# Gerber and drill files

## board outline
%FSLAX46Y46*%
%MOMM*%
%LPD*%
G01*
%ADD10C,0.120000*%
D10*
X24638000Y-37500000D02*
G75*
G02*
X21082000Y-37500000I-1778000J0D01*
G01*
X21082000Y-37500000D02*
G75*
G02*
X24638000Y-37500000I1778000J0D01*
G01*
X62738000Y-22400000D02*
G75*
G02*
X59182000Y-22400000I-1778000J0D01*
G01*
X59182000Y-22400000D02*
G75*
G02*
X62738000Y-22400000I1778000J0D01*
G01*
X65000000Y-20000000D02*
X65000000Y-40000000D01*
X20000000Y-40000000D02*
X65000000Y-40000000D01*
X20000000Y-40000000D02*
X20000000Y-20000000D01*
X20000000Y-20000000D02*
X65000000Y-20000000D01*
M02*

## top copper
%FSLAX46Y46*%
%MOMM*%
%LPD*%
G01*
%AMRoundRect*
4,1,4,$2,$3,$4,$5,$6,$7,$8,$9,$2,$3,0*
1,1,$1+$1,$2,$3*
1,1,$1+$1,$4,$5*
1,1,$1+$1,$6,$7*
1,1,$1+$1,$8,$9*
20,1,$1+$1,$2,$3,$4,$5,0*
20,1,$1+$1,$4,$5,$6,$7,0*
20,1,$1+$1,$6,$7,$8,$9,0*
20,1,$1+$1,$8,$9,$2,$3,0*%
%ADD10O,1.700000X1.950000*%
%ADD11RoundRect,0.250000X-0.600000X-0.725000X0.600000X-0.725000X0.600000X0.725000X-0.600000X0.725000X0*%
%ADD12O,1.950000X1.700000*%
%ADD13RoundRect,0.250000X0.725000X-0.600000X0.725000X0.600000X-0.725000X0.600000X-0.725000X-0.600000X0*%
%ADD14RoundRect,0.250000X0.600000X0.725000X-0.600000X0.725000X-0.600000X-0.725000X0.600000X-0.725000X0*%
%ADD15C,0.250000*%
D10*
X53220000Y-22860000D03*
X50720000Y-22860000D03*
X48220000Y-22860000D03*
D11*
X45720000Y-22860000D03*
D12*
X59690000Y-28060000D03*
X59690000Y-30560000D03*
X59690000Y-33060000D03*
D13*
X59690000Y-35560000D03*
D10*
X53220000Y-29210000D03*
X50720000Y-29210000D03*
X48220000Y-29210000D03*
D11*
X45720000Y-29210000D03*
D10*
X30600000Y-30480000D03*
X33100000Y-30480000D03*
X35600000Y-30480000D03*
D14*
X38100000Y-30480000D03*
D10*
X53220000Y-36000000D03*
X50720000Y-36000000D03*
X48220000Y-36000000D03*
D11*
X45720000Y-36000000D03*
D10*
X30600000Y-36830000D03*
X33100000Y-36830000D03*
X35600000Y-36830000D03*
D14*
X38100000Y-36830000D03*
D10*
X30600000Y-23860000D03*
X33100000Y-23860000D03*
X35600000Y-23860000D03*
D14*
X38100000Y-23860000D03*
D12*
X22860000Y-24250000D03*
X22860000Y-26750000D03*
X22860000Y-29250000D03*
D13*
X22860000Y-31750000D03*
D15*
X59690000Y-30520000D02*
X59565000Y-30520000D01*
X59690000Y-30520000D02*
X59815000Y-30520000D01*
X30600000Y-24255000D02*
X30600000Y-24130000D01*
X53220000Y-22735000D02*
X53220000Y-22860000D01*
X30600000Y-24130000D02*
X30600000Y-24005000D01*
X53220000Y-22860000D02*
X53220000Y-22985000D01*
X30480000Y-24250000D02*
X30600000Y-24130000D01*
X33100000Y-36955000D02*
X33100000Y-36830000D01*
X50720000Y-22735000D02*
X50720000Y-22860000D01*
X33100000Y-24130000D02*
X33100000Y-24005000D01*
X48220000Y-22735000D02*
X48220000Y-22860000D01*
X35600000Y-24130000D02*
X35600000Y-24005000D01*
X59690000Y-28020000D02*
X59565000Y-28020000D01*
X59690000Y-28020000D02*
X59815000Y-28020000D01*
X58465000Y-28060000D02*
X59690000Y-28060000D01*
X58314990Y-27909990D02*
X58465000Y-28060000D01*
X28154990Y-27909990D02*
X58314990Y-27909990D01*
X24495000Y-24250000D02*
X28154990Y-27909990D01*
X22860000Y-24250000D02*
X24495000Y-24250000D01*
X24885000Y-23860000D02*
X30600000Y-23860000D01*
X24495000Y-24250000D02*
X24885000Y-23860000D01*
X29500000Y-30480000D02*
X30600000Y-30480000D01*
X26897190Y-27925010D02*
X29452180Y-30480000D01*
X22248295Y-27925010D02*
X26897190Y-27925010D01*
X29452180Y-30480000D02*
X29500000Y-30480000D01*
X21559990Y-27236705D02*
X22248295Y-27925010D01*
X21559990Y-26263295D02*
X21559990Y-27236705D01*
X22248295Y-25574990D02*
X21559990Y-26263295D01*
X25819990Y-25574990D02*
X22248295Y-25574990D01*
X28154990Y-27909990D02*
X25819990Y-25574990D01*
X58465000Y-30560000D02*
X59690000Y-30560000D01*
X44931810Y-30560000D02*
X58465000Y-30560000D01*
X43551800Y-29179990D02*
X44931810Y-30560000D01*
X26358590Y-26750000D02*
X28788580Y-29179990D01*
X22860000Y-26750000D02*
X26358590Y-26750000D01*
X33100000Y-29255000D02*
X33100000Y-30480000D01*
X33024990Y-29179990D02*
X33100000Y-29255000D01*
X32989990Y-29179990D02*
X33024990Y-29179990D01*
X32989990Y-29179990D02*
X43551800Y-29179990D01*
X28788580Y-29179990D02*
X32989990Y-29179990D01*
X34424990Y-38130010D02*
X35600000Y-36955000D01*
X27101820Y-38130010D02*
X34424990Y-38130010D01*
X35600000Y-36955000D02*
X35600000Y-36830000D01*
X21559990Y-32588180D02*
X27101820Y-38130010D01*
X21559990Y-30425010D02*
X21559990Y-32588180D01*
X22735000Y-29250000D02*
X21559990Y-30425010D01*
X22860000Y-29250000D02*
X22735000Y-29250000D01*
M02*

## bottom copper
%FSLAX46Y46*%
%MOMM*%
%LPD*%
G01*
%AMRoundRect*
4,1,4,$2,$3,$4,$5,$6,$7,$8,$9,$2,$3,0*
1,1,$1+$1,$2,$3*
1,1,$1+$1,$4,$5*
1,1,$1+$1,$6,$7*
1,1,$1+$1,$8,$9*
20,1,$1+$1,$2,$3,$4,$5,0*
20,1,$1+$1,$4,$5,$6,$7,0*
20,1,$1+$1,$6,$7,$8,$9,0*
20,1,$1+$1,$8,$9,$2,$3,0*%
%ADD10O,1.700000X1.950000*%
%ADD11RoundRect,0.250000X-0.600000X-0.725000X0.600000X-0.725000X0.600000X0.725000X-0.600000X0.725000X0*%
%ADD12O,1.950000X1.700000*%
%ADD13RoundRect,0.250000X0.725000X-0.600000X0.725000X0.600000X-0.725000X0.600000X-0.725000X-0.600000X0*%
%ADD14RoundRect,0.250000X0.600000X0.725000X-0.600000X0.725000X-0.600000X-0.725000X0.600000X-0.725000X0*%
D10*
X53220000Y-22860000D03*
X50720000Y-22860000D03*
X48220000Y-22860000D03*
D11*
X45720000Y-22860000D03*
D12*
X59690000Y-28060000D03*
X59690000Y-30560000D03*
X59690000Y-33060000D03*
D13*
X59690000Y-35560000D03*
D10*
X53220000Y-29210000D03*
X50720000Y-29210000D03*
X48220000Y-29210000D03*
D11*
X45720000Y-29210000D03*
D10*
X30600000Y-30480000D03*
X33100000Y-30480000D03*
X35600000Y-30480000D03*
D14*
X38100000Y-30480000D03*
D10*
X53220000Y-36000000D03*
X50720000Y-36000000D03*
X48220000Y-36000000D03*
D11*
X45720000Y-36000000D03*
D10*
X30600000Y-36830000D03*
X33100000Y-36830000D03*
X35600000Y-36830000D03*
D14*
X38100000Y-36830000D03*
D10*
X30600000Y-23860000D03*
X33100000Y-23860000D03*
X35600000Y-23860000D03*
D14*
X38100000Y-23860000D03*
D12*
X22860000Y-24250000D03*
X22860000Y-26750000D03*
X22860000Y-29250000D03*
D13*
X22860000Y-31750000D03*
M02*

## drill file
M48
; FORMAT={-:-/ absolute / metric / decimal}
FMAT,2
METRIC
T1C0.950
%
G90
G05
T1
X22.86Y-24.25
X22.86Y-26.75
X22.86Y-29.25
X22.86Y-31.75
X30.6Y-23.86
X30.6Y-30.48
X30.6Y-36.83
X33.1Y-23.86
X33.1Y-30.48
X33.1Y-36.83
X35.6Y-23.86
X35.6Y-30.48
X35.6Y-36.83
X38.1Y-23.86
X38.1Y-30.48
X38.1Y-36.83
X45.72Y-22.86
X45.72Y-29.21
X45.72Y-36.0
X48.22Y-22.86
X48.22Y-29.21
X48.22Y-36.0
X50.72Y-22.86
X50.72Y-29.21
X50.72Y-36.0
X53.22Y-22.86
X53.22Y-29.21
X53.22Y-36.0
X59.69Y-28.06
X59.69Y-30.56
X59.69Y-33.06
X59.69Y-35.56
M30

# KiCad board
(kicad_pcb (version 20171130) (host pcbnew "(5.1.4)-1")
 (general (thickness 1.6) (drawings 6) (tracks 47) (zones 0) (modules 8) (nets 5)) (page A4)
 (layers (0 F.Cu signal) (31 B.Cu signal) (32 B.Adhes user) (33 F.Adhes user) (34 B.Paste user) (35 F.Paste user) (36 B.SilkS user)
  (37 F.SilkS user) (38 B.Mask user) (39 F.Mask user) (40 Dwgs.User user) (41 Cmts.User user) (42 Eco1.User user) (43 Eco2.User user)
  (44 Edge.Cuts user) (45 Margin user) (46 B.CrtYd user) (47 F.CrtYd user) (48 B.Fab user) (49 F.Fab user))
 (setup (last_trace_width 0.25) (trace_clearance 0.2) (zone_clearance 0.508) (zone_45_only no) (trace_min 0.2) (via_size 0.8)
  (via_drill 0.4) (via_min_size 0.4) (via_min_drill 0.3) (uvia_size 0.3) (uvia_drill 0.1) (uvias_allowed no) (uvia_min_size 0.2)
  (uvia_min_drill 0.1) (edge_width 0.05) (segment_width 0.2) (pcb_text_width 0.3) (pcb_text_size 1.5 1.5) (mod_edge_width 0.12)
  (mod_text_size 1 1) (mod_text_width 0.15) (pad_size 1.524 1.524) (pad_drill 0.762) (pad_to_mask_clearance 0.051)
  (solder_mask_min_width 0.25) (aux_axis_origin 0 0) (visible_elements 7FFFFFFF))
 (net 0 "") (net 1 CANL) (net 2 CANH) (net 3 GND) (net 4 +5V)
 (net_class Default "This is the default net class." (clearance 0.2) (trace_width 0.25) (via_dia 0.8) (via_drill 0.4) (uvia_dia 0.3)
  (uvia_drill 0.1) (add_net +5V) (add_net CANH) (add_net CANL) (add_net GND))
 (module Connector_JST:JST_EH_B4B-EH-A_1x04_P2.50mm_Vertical (layer F.Cu) (at 45.72 22.86)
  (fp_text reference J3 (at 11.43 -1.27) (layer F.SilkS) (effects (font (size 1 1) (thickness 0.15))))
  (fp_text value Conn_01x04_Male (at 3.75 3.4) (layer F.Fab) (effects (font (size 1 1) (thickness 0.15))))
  (pad 4 thru_hole oval (at 7.5 0) (size 1.7 1.95) (drill 0.95) (layers *.Cu *.Mask) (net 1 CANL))
  (pad 3 thru_hole oval (at 5 0) (size 1.7 1.95) (drill 0.95) (layers *.Cu *.Mask) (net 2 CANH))
  (pad 2 thru_hole oval (at 2.5 0) (size 1.7 1.95) (drill 0.95) (layers *.Cu *.Mask) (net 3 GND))
  (pad 1 thru_hole roundrect (at 0 0) (size 1.7 1.95) (drill 0.95) (layers *.Cu *.Mask) (roundrect_rratio 0.147059) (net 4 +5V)))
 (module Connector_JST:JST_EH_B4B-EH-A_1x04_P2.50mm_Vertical (layer F.Cu) (at 59.69 35.56 90)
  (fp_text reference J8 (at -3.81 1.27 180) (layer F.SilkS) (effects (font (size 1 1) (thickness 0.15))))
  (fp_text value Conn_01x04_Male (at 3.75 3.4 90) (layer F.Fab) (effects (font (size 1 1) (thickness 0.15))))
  (pad 4 thru_hole oval (at 7.5 0 90) (size 1.7 1.95) (drill 0.95) (layers *.Cu *.Mask) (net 1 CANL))
  (pad 3 thru_hole oval (at 5 0 90) (size 1.7 1.95) (drill 0.95) (layers *.Cu *.Mask) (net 2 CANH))
  (pad 2 thru_hole oval (at 2.5 0 90) (size 1.7 1.95) (drill 0.95) (layers *.Cu *.Mask) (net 3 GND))
  (pad 1 thru_hole roundrect (at 0 0 90) (size 1.7 1.95) (drill 0.95) (layers *.Cu *.Mask) (roundrect_rratio 0.147059) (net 4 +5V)))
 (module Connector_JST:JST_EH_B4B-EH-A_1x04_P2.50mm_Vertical (layer F.Cu) (at 45.72 29.21)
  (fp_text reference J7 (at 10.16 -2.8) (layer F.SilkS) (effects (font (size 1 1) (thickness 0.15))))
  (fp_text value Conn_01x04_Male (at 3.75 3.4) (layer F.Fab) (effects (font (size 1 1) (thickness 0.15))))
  (pad 4 thru_hole oval (at 7.5 0) (size 1.7 1.95) (drill 0.95) (layers *.Cu *.Mask) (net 1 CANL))
  (pad 3 thru_hole oval (at 5 0) (size 1.7 1.95) (drill 0.95) (layers *.Cu *.Mask) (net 2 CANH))
  (pad 2 thru_hole oval (at 2.5 0) (size 1.7 1.95) (drill 0.95) (layers *.Cu *.Mask) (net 3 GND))
  (pad 1 thru_hole roundrect (at 0 0) (size 1.7 1.95) (drill 0.95) (layers *.Cu *.Mask) (roundrect_rratio 0.147059) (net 4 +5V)))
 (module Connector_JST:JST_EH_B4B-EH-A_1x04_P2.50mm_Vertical (layer F.Cu) (at 38.1 30.48 180)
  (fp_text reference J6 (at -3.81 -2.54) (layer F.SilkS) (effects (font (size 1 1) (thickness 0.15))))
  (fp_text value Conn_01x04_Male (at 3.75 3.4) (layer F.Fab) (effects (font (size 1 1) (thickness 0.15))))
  (pad 4 thru_hole oval (at 7.5 0 180) (size 1.7 1.95) (drill 0.95) (layers *.Cu *.Mask) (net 1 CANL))
  (pad 3 thru_hole oval (at 5 0 180) (size 1.7 1.95) (drill 0.95) (layers *.Cu *.Mask) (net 2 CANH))
  (pad 2 thru_hole oval (at 2.5 0 180) (size 1.7 1.95) (drill 0.95) (layers *.Cu *.Mask) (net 3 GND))
  (pad 1 thru_hole roundrect (at 0 0 180) (size 1.7 1.95) (drill 0.95) (layers *.Cu *.Mask) (roundrect_rratio 0.147059) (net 4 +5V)))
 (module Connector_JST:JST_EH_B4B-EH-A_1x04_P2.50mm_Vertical (layer F.Cu) (at 45.72 36)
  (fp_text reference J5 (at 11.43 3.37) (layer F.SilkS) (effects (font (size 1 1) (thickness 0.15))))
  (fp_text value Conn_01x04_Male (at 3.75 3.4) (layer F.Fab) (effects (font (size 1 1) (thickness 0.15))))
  (pad 4 thru_hole oval (at 7.5 0) (size 1.7 1.95) (drill 0.95) (layers *.Cu *.Mask) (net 1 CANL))
  (pad 3 thru_hole oval (at 5 0) (size 1.7 1.95) (drill 0.95) (layers *.Cu *.Mask) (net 2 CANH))
  (pad 2 thru_hole oval (at 2.5 0) (size 1.7 1.95) (drill 0.95) (layers *.Cu *.Mask) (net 3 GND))
  (pad 1 thru_hole roundrect (at 0 0) (size 1.7 1.95) (drill 0.95) (layers *.Cu *.Mask) (roundrect_rratio 0.147059) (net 4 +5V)))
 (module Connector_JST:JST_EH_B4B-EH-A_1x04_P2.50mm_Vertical (layer F.Cu) (at 38.1 36.83 180)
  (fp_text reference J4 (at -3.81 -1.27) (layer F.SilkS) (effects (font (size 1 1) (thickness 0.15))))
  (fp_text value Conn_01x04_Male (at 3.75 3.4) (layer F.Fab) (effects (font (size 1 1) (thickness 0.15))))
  (pad 4 thru_hole oval (at 7.5 0 180) (size 1.7 1.95) (drill 0.95) (layers *.Cu *.Mask) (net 1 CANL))
  (pad 3 thru_hole oval (at 5 0 180) (size 1.7 1.95) (drill 0.95) (layers *.Cu *.Mask) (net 2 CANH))
  (pad 2 thru_hole oval (at 2.5 0 180) (size 1.7 1.95) (drill 0.95) (layers *.Cu *.Mask) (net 3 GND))
  (pad 1 thru_hole roundrect (at 0 0 180) (size 1.7 1.95) (drill 0.95) (layers *.Cu *.Mask) (roundrect_rratio 0.147059) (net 4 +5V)))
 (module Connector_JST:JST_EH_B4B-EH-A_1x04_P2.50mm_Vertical (layer F.Cu) (at 38.1 23.86 180)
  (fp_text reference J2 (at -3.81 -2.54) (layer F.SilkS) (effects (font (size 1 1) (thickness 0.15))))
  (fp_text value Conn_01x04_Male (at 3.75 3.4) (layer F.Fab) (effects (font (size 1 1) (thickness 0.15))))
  (pad 4 thru_hole oval (at 7.5 0 180) (size 1.7 1.95) (drill 0.95) (layers *.Cu *.Mask) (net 1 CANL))
  (pad 3 thru_hole oval (at 5 0 180) (size 1.7 1.95) (drill 0.95) (layers *.Cu *.Mask) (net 2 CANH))
  (pad 2 thru_hole oval (at 2.5 0 180) (size 1.7 1.95) (drill 0.95) (layers *.Cu *.Mask) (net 3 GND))
  (pad 1 thru_hole roundrect (at 0 0 180) (size 1.7 1.95) (drill 0.95) (layers *.Cu *.Mask) (roundrect_rratio 0.147059) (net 4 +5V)))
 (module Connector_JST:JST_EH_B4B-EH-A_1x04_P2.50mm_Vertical (layer F.Cu) (at 22.86 31.75 90)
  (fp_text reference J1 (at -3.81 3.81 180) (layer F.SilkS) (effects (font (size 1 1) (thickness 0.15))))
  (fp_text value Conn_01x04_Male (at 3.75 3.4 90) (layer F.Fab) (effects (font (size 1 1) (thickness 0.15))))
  (pad 4 thru_hole oval (at 7.5 0 90) (size 1.7 1.95) (drill 0.95) (layers *.Cu *.Mask) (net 1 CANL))
  (pad 3 thru_hole oval (at 5 0 90) (size 1.7 1.95) (drill 0.95) (layers *.Cu *.Mask) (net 2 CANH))
  (pad 2 thru_hole oval (at 2.5 0 90) (size 1.7 1.95) (drill 0.95) (layers *.Cu *.Mask) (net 3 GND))
  (pad 1 thru_hole roundrect (at 0 0 90) (size 1.7 1.95) (drill 0.95) (layers *.Cu *.Mask) (roundrect_rratio 0.147059) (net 4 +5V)))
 (gr_circle (center 22.86 37.5) (end 24.638 37.5) (layer Edge.Cuts) (width 0.12))
 (gr_circle (center 60.96 22.4) (end 62.738 22.4) (layer Edge.Cuts) (width 0.12))
 (gr_line (start 65 20) (end 65 40) (layer Edge.Cuts) (width 0.12))
 (gr_line (start 20 40) (end 65 40) (layer Edge.Cuts) (width 0.12))
 (gr_line (start 20 40) (end 20 20) (layer Edge.Cuts) (width 0.12))
 (gr_line (start 20 20) (end 65 20) (layer Edge.Cuts) (width 0.12))
 (segment (start 59.69 30.52) (end 59.565 30.52) (width 0.25) (layer F.Cu) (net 2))
 (segment (start 59.69 30.52) (end 59.815 30.52) (width 0.25) (layer F.Cu) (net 2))
 (segment (start 30.6 24.255) (end 30.6 24.13) (width 0.25) (layer F.Cu) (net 1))
 (segment (start 53.22 22.735) (end 53.22 22.86) (width 0.25) (layer F.Cu) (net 1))
 (segment (start 30.6 24.13) (end 30.6 24.005) (width 0.25) (layer F.Cu) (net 1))
 (segment (start 53.22 22.86) (end 53.22 22.985) (width 0.25) (layer F.Cu) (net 1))
 (segment (start 30.48 24.25) (end 30.6 24.13) (width 0.25) (layer F.Cu) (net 1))
 (segment (start 33.1 36.955) (end 33.1 36.83) (width 0.25) (layer F.Cu) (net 2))
 (segment (start 50.72 22.735) (end 50.72 22.86) (width 0.25) (layer F.Cu) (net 2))
 (segment (start 33.1 24.13) (end 33.1 24.005) (width 0.25) (layer F.Cu) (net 2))
 (segment (start 48.22 22.735) (end 48.22 22.86) (width 0.25) (layer F.Cu) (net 3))
 (segment (start 35.6 24.13) (end 35.6 24.005) (width 0.25) (layer F.Cu) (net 3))
 (segment (start 59.69 28.02) (end 59.565 28.02) (width 0.25) (layer F.Cu) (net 1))
 (segment (start 59.69 28.02) (end 59.815 28.02) (width 0.25) (layer F.Cu) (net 1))
 (segment (start 58.465 28.06) (end 59.69 28.06) (width 0.25) (layer F.Cu) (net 1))
 (segment (start 58.31499 27.90999) (end 58.465 28.06) (width 0.25) (layer F.Cu) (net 1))
 (segment (start 28.15499 27.90999) (end 58.31499 27.90999) (width 0.25) (layer F.Cu) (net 1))
 (segment (start 24.495 24.25) (end 28.15499 27.90999) (width 0.25) (layer F.Cu) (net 1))
 (segment (start 22.86 24.25) (end 24.495 24.25) (width 0.25) (layer F.Cu) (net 1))
 (segment (start 24.885 23.86) (end 30.6 23.86) (width 0.25) (layer F.Cu) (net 1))
 (segment (start 24.495 24.25) (end 24.885 23.86) (width 0.25) (layer F.Cu) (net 1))
 (segment (start 29.5 30.48) (end 30.6 30.48) (width 0.25) (layer F.Cu) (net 1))
 (segment (start 26.89719 27.92501) (end 29.45218 30.48) (width 0.25) (layer F.Cu) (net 1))
 (segment (start 22.248295 27.92501) (end 26.89719 27.92501) (width 0.25) (layer F.Cu) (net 1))
 (segment (start 29.45218 30.48) (end 29.5 30.48) (width 0.25) (layer F.Cu) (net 1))
 (segment (start 21.55999 27.236705) (end 22.248295 27.92501) (width 0.25) (layer F.Cu) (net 1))
 (segment (start 21.55999 26.263295) (end 21.55999 27.236705) (width 0.25) (layer F.Cu) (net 1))
 (segment (start 22.248295 25.57499) (end 21.55999 26.263295) (width 0.25) (layer F.Cu) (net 1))
 (segment (start 25.81999 25.57499) (end 22.248295 25.57499) (width 0.25) (layer F.Cu) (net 1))
 (segment (start 28.15499 27.90999) (end 25.81999 25.57499) (width 0.25) (layer F.Cu) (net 1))
 (segment (start 58.465 30.56) (end 59.69 30.56) (width 0.25) (layer F.Cu) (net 2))
 (segment (start 44.93181 30.56) (end 58.465 30.56) (width 0.25) (layer F.Cu) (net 2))
 (segment (start 43.5518 29.17999) (end 44.93181 30.56) (width 0.25) (layer F.Cu) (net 2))
 (segment (start 26.35859 26.75) (end 28.78858 29.17999) (width 0.25) (layer F.Cu) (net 2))
 (segment (start 22.86 26.75) (end 26.35859 26.75) (width 0.25) (layer F.Cu) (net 2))
 (segment (start 33.1 29.255) (end 33.1 30.48) (width 0.25) (layer F.Cu) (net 2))
 (segment (start 33.02499 29.17999) (end 33.1 29.255) (width 0.25) (layer F.Cu) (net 2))
 (segment (start 32.98999 29.17999) (end 33.02499 29.17999) (width 0.25) (layer F.Cu) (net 2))
 (segment (start 32.98999 29.17999) (end 43.5518 29.17999) (width 0.25) (layer F.Cu) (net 2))
 (segment (start 28.78858 29.17999) (end 32.98999 29.17999) (width 0.25) (layer F.Cu) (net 2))
 (segment (start 34.42499 38.13001) (end 35.6 36.955) (width 0.25) (layer F.Cu) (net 3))
 (segment (start 27.10182 38.13001) (end 34.42499 38.13001) (width 0.25) (layer F.Cu) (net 3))
 (segment (start 35.6 36.955) (end 35.6 36.83) (width 0.25) (layer F.Cu) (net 3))
 (segment (start 21.55999 32.58818) (end 27.10182 38.13001) (width 0.25) (layer F.Cu) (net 3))
 (segment (start 21.55999 30.42501) (end 21.55999 32.58818) (width 0.25) (layer F.Cu) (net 3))
 (segment (start 22.735 29.25) (end 21.55999 30.42501) (width 0.25) (layer F.Cu) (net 3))
 (segment (start 22.86 29.25) (end 22.735 29.25) (width 0.25) (layer F.Cu) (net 3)))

